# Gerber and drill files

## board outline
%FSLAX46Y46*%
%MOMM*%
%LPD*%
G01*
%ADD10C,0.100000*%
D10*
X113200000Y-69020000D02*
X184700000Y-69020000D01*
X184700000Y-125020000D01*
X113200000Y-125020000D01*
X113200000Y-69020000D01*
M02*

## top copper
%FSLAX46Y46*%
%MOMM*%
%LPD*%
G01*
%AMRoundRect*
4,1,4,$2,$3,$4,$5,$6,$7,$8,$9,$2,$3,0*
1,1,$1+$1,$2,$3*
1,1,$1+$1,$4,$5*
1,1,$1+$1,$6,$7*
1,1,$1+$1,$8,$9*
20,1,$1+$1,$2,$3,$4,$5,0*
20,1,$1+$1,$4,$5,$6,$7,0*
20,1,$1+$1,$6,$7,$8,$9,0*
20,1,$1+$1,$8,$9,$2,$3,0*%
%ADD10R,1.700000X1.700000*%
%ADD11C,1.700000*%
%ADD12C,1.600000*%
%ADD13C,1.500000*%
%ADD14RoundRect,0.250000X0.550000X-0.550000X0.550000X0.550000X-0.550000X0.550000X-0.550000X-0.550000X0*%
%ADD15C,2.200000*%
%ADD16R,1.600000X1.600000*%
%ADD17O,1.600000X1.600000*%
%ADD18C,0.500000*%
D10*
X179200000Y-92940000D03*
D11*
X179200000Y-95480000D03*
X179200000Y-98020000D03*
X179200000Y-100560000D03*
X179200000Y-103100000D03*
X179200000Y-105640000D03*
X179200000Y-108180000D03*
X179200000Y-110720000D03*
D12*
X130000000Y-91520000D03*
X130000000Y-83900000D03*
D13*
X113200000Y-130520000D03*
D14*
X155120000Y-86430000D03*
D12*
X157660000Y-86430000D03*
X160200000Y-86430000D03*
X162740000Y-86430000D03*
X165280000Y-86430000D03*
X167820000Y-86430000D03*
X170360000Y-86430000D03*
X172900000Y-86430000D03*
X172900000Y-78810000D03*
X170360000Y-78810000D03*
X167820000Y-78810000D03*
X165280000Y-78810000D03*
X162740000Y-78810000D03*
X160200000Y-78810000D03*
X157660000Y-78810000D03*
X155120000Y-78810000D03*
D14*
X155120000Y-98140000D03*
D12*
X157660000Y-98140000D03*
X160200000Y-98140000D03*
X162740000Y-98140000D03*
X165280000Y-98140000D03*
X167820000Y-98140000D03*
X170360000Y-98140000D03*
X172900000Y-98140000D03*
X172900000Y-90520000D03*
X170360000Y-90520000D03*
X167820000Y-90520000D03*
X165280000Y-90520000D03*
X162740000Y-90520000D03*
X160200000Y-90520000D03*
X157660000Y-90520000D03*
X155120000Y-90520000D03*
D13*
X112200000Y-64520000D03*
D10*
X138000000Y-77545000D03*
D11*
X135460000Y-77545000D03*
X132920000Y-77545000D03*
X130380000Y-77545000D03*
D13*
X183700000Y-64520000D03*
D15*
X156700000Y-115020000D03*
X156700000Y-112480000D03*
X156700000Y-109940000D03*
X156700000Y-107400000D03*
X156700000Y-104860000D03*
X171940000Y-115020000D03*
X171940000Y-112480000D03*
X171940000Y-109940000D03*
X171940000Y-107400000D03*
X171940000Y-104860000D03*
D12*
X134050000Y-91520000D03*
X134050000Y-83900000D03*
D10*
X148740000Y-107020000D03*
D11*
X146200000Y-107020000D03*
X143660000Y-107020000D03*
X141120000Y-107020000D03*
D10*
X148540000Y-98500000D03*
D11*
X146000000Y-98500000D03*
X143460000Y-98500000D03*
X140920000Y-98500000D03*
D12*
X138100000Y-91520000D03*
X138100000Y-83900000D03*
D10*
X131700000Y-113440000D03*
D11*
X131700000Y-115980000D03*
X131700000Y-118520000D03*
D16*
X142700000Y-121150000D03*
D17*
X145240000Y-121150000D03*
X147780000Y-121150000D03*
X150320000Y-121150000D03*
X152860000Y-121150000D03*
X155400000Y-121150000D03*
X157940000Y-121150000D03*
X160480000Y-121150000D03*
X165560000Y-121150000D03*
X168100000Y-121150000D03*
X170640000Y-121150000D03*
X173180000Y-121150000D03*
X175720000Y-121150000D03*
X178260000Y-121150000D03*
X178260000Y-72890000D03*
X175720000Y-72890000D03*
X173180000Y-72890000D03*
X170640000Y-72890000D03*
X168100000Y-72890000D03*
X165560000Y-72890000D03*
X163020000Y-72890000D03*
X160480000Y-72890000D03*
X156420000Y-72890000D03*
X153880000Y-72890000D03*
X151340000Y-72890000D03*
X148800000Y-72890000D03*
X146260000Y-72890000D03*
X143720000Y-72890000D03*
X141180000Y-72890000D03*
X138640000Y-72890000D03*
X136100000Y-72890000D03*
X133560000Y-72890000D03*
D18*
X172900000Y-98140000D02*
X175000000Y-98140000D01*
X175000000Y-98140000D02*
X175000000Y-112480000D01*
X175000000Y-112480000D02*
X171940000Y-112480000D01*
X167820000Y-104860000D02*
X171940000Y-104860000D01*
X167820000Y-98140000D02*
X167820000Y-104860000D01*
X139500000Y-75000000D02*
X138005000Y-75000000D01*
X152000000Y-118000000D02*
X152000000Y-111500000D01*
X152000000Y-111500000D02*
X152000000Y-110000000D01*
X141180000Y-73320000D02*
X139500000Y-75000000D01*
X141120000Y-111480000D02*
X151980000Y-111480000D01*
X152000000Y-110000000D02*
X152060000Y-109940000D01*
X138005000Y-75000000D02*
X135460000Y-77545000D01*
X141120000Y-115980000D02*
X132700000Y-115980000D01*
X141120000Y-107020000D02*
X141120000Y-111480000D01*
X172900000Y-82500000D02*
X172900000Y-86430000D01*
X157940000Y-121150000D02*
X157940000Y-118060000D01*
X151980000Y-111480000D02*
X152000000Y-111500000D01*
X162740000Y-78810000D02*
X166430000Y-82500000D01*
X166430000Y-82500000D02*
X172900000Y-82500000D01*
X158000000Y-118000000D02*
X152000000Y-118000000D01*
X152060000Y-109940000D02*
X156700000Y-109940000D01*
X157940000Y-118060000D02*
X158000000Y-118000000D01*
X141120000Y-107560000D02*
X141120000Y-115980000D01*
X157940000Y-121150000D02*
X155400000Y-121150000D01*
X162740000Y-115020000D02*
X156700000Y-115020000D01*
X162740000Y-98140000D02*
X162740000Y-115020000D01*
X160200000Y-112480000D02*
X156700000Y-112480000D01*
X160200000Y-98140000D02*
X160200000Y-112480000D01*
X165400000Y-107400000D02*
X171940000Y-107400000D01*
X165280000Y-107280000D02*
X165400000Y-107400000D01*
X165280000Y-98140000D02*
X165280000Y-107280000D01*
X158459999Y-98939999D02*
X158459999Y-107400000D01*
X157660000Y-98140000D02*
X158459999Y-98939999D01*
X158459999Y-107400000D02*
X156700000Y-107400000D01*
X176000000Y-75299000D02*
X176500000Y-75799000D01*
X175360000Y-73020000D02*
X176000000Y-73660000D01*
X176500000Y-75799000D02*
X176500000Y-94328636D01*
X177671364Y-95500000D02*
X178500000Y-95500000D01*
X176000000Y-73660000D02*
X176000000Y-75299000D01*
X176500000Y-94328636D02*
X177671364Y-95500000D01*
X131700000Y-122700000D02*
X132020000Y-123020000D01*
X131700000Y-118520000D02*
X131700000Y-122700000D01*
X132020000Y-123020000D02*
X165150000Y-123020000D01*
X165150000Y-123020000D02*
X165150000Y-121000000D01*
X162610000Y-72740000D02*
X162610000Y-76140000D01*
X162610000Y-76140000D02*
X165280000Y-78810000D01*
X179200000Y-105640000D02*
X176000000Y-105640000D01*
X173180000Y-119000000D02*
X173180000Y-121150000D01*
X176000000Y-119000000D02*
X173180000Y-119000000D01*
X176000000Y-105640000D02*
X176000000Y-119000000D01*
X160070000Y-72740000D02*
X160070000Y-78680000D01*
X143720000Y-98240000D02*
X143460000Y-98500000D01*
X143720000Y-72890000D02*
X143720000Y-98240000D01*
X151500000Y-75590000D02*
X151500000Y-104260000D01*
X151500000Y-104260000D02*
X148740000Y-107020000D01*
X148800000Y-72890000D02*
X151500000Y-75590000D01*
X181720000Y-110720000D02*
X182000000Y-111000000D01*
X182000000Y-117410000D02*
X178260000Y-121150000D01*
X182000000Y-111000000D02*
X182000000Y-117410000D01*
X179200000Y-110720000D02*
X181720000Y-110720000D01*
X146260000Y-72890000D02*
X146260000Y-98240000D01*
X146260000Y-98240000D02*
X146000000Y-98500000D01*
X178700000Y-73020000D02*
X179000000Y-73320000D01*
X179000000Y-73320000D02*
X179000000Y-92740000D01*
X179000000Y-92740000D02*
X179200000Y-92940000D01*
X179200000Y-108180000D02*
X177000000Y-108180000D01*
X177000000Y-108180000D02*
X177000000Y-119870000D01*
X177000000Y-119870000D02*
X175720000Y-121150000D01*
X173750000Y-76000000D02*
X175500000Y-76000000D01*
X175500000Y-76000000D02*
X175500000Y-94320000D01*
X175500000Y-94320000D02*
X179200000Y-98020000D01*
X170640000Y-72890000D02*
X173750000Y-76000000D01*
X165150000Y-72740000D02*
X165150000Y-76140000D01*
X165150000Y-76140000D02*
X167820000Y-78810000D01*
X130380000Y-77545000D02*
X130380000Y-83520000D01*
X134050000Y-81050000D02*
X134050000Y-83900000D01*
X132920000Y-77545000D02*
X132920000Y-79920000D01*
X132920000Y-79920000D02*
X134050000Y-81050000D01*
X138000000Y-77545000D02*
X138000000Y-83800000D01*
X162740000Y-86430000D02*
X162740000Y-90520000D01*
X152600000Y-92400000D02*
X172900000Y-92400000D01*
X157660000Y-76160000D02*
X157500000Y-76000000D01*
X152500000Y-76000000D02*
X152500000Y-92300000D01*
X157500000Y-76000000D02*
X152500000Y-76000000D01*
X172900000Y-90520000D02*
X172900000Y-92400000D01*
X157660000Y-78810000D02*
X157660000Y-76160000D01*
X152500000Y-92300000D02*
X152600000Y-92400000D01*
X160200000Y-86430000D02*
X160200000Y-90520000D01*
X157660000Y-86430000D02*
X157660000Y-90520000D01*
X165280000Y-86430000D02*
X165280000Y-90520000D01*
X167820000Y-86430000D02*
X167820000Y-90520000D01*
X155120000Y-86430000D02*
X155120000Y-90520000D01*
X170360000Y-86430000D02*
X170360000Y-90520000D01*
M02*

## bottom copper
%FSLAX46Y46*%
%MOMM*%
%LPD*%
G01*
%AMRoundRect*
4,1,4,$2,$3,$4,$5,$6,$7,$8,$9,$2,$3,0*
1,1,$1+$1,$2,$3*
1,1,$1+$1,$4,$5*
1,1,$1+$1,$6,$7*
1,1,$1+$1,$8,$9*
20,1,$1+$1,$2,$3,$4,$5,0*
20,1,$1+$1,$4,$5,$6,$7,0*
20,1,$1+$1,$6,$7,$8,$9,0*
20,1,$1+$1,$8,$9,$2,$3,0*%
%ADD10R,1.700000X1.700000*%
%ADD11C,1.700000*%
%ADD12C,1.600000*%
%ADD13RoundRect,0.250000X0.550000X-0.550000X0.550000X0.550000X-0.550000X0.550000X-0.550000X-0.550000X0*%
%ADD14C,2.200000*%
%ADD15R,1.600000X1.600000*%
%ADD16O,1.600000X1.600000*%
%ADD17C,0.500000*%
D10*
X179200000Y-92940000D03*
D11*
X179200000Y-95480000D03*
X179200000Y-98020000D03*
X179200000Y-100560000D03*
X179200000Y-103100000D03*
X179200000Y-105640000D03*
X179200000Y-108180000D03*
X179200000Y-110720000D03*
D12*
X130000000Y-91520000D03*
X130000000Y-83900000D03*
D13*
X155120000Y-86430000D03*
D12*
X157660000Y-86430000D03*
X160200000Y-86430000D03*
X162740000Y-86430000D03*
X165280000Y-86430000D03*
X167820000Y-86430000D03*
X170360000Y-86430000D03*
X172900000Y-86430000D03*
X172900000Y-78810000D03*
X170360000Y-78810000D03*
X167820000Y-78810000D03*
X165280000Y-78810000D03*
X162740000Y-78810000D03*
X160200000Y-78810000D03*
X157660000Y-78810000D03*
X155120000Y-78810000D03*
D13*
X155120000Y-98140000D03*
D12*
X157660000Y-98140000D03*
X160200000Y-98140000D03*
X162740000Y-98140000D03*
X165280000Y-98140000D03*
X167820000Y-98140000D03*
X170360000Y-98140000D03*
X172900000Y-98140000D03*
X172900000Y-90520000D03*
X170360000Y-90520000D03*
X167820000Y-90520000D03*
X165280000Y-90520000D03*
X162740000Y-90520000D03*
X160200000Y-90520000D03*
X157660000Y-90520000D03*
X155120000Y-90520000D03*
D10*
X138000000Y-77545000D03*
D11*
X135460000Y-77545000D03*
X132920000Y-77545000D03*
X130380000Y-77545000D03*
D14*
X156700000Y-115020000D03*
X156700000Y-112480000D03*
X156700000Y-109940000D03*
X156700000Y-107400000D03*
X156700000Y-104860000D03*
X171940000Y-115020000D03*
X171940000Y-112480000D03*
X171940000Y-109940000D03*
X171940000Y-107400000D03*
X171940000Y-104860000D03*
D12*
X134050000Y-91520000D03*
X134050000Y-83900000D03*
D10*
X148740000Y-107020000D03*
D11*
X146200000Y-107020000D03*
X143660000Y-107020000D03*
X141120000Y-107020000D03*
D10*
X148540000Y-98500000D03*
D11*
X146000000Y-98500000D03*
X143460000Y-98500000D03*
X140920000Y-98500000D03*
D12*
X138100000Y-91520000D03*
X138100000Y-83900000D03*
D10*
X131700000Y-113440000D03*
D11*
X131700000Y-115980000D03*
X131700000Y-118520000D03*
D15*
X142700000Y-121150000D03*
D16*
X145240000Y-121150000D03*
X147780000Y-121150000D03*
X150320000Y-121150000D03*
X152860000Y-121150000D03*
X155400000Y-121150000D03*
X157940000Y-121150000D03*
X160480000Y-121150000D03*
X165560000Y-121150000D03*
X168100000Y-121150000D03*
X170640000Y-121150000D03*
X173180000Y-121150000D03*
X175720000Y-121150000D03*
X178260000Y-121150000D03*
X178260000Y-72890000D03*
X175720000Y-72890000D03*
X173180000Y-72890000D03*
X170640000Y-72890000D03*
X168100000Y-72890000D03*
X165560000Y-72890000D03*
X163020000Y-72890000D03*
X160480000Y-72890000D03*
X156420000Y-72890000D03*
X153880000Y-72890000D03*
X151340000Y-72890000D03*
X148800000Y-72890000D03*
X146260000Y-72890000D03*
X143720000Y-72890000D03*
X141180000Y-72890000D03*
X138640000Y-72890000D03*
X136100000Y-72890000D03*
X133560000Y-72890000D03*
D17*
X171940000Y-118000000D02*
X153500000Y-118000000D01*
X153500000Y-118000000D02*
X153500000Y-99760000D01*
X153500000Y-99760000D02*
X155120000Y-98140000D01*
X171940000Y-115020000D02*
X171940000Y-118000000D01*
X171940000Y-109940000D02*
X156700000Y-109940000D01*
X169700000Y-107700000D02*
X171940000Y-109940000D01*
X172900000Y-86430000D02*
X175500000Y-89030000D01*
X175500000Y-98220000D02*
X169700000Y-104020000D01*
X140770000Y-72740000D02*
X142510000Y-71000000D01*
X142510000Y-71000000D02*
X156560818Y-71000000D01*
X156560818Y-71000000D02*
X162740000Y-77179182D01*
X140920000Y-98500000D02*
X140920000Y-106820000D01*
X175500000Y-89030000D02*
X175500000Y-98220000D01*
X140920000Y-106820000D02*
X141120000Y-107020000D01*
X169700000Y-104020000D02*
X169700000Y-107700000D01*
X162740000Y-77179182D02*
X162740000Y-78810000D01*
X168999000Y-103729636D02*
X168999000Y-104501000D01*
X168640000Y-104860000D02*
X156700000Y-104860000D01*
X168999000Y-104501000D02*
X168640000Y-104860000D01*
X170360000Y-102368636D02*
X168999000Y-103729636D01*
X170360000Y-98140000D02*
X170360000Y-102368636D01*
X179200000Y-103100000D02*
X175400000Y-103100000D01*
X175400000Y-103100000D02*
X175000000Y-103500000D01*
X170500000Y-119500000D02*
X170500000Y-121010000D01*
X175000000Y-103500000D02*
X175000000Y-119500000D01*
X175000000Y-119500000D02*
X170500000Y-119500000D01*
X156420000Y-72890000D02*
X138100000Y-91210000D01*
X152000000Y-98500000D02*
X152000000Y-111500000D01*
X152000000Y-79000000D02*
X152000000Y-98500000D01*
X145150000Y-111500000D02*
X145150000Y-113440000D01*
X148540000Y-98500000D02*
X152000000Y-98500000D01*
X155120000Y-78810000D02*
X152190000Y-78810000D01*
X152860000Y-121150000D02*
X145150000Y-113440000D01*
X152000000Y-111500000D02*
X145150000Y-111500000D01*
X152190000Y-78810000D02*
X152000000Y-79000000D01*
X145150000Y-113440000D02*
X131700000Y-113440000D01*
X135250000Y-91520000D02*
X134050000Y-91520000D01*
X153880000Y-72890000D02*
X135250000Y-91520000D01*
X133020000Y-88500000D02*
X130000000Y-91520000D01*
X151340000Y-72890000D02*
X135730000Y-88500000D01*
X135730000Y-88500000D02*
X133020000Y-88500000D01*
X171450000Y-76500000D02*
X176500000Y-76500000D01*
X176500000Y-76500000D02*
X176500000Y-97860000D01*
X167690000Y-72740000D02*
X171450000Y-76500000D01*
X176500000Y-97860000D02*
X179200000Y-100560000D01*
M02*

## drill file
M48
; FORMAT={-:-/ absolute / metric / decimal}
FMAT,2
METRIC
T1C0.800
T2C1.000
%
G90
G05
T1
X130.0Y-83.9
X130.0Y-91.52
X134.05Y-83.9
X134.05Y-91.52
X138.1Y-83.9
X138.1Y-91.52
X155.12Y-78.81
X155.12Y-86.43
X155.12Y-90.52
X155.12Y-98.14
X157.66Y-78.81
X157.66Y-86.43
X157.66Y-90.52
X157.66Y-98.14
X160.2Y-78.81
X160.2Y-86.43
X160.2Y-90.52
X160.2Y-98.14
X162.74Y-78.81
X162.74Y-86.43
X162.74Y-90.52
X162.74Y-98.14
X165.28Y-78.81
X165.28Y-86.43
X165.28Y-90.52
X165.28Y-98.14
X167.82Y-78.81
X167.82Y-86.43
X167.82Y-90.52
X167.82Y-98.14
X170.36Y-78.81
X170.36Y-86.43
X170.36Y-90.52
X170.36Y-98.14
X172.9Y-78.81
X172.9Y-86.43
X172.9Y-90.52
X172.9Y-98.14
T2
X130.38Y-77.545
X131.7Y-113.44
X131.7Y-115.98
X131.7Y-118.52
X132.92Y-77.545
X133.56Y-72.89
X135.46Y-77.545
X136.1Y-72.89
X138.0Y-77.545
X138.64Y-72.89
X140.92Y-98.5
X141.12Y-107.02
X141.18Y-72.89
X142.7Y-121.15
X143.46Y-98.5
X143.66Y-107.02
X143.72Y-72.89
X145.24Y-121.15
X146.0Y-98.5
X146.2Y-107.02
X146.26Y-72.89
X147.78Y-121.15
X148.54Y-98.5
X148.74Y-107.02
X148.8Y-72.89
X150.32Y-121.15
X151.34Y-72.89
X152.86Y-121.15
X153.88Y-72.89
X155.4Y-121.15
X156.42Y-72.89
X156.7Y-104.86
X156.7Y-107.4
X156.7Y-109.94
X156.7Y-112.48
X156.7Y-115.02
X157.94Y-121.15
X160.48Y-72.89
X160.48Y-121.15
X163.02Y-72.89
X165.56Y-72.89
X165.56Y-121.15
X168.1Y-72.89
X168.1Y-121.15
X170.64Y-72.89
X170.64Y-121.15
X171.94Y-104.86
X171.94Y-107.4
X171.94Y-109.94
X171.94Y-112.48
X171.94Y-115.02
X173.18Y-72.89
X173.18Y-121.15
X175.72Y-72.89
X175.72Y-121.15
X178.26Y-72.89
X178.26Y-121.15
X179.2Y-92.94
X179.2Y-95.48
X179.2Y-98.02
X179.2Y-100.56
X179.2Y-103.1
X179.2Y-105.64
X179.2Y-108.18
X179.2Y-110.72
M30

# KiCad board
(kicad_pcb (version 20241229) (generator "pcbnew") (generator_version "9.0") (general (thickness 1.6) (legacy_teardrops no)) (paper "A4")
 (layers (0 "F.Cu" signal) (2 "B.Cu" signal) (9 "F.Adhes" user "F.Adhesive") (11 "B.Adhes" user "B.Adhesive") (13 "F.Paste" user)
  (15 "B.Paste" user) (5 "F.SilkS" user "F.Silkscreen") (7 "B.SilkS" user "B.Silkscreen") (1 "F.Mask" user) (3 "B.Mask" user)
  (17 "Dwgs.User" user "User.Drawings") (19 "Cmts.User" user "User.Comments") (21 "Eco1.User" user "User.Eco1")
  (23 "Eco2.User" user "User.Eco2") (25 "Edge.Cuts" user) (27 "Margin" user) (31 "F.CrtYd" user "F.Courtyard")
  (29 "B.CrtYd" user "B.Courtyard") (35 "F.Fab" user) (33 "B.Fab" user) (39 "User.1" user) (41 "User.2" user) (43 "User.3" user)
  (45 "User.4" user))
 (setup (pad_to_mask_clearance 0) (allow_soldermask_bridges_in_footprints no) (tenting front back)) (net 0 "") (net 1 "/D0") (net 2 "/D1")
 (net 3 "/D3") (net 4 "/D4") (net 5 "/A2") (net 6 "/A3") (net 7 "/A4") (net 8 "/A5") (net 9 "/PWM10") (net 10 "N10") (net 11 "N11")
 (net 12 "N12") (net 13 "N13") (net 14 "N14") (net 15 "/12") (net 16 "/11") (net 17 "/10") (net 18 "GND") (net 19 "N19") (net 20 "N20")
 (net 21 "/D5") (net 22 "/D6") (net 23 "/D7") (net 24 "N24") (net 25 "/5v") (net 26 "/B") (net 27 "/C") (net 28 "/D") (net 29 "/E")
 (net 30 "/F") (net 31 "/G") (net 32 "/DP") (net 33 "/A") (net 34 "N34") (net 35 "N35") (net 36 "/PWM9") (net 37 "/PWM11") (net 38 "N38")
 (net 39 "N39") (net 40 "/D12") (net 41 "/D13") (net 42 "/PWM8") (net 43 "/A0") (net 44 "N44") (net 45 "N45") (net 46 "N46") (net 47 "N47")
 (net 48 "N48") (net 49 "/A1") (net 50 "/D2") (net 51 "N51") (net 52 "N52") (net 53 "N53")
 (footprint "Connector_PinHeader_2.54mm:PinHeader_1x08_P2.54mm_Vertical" (layer "F.Cu") (at 179.2 92.94)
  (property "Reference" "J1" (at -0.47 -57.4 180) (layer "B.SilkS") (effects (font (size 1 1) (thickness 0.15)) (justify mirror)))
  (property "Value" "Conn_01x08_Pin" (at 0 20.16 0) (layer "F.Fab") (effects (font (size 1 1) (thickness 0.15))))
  (pad "1" thru_hole rect (at 0 0) (size 1.7 1.7) (drill 1) (layers "*.Cu" "*.Mask") (remove_unused_layers no) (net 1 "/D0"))
  (pad "2" thru_hole circle (at 0 2.54) (size 1.7 1.7) (drill 1) (layers "*.Cu" "*.Mask") (remove_unused_layers no) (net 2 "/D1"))
  (pad "3" thru_hole circle (at 0 5.08) (size 1.7 1.7) (drill 1) (layers "*.Cu" "*.Mask") (remove_unused_layers no) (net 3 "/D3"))
  (pad "4" thru_hole circle (at 0 7.62) (size 1.7 1.7) (drill 1) (layers "*.Cu" "*.Mask") (remove_unused_layers no) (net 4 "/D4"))
  (pad "5" thru_hole circle (at 0 10.16) (size 1.7 1.7) (drill 1) (layers "*.Cu" "*.Mask") (remove_unused_layers no) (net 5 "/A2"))
  (pad "6" thru_hole circle (at 0 12.7) (size 1.7 1.7) (drill 1) (layers "*.Cu" "*.Mask") (remove_unused_layers no) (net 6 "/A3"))
  (pad "7" thru_hole circle (at 0 15.24) (size 1.7 1.7) (drill 1) (layers "*.Cu" "*.Mask") (remove_unused_layers no) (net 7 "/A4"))
  (pad "8" thru_hole circle (at 0 17.78) (size 1.7 1.7) (drill 1) (layers "*.Cu" "*.Mask") (remove_unused_layers no) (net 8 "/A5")))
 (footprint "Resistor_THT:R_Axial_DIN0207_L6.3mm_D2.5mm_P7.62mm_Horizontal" (layer "F.Cu") (at 130 91.52 90)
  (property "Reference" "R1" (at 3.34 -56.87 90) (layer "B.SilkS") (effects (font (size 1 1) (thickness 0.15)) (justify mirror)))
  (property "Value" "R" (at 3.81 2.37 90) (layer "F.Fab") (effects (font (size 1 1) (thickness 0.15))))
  (pad "1" thru_hole circle (at 0 0 90) (size 1.6 1.6) (drill 0.8) (layers "*.Cu" "*.Mask") (remove_unused_layers no) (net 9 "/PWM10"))
  (pad "2" thru_hole circle (at 7.62 0 90) (size 1.6 1.6) (drill 0.8) (layers "*.Cu" "*.Mask") (remove_unused_layers no) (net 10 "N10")))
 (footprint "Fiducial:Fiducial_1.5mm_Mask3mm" (layer "F.Cu") (at 113.2 130.52)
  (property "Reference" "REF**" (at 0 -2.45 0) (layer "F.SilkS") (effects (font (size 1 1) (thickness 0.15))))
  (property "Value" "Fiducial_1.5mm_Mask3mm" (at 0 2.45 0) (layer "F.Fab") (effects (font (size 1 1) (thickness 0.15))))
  (pad "" smd circle (at 0 0) (size 1.5 1.5) (layers "F.Cu" "F.Mask") (solder_mask_margin 0.75)))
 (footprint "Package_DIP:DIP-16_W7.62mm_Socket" (layer "F.Cu") (at 155.12 86.43 90)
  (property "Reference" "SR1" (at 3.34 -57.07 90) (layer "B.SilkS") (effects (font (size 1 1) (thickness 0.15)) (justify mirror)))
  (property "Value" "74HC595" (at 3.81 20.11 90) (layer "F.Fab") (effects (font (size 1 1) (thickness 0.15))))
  (pad "1" thru_hole roundrect (at 0 0 90) (size 1.6 1.6) (drill 0.8) (layers "*.Cu" "*.Mask") (remove_unused_layers no)
   (roundrect_rratio 0.15625) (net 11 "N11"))
  (pad "2" thru_hole circle (at 0 2.54 90) (size 1.6 1.6) (drill 0.8) (layers "*.Cu" "*.Mask") (remove_unused_layers no) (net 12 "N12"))
  (pad "3" thru_hole circle (at 0 5.08 90) (size 1.6 1.6) (drill 0.8) (layers "*.Cu" "*.Mask") (remove_unused_layers no) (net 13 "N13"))
  (pad "4" thru_hole circle (at 0 7.62 90) (size 1.6 1.6) (drill 0.8) (layers "*.Cu" "*.Mask") (remove_unused_layers no) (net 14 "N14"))
  (pad "5" thru_hole circle (at 0 10.16 90) (size 1.6 1.6) (drill 0.8) (layers "*.Cu" "*.Mask") (remove_unused_layers no) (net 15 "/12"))
  (pad "6" thru_hole circle (at 0 12.7 90) (size 1.6 1.6) (drill 0.8) (layers "*.Cu" "*.Mask") (remove_unused_layers no) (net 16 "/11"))
  (pad "7" thru_hole circle (at 0 15.24 90) (size 1.6 1.6) (drill 0.8) (layers "*.Cu" "*.Mask") (remove_unused_layers no) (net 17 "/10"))
  (pad "8" thru_hole circle (at 0 17.78 90) (size 1.6 1.6) (drill 0.8) (layers "*.Cu" "*.Mask") (remove_unused_layers no) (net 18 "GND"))
  (pad "9" thru_hole circle (at 7.62 17.78 90) (size 1.6 1.6) (drill 0.8) (layers "*.Cu" "*.Mask") (remove_unused_layers no) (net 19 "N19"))
  (pad "10" thru_hole circle (at 7.62 15.24 90) (size 1.6 1.6) (drill 0.8) (layers "*.Cu" "*.Mask") (remove_unused_layers no) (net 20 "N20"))
  (pad "11" thru_hole circle (at 7.62 12.7 90) (size 1.6 1.6) (drill 0.8) (layers "*.Cu" "*.Mask") (remove_unused_layers no) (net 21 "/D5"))
  (pad "12" thru_hole circle (at 7.62 10.16 90) (size 1.6 1.6) (drill 0.8) (layers "*.Cu" "*.Mask") (remove_unused_layers no) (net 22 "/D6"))
  (pad "13" thru_hole circle (at 7.62 7.62 90) (size 1.6 1.6) (drill 0.8) (layers "*.Cu" "*.Mask") (remove_unused_layers no) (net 18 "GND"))
  (pad "14" thru_hole circle (at 7.62 5.08 90) (size 1.6 1.6) (drill 0.8) (layers "*.Cu" "*.Mask") (remove_unused_layers no) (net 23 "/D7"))
  (pad "15" thru_hole circle (at 7.62 2.54 90) (size 1.6 1.6) (drill 0.8) (layers "*.Cu" "*.Mask") (remove_unused_layers no) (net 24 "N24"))
  (pad "16" thru_hole circle (at 7.62 0 90) (size 1.6 1.6) (drill 0.8) (layers "*.Cu" "*.Mask") (remove_unused_layers no) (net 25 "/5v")))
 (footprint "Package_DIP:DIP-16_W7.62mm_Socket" (layer "F.Cu") (at 155.12 98.14 90)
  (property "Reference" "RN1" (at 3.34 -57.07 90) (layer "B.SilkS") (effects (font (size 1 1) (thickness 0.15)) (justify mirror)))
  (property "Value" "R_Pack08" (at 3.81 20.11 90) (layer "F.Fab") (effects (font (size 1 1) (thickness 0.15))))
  (pad "1" thru_hole roundrect (at 0 0 90) (size 1.6 1.6) (drill 0.8) (layers "*.Cu" "*.Mask") (remove_unused_layers no)
   (roundrect_rratio 0.15625) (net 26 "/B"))
  (pad "2" thru_hole circle (at 0 2.54 90) (size 1.6 1.6) (drill 0.8) (layers "*.Cu" "*.Mask") (remove_unused_layers no) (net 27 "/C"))
  (pad "3" thru_hole circle (at 0 5.08 90) (size 1.6 1.6) (drill 0.8) (layers "*.Cu" "*.Mask") (remove_unused_layers no) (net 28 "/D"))
  (pad "4" thru_hole circle (at 0 7.62 90) (size 1.6 1.6) (drill 0.8) (layers "*.Cu" "*.Mask") (remove_unused_layers no) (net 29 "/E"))
  (pad "5" thru_hole circle (at 0 10.16 90) (size 1.6 1.6) (drill 0.8) (layers "*.Cu" "*.Mask") (remove_unused_layers no) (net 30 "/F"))
  (pad "6" thru_hole circle (at 0 12.7 90) (size 1.6 1.6) (drill 0.8) (layers "*.Cu" "*.Mask") (remove_unused_layers no) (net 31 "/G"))
  (pad "7" thru_hole circle (at 0 15.24 90) (size 1.6 1.6) (drill 0.8) (layers "*.Cu" "*.Mask") (remove_unused_layers no) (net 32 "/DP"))
  (pad "8" thru_hole circle (at 0 17.78 90) (size 1.6 1.6) (drill 0.8) (layers "*.Cu" "*.Mask") (remove_unused_layers no) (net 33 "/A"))
  (pad "9" thru_hole circle (at 7.62 17.78 90) (size 1.6 1.6) (drill 0.8) (layers "*.Cu" "*.Mask") (remove_unused_layers no) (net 24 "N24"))
  (pad "10" thru_hole circle (at 7.62 15.24 90) (size 1.6 1.6) (drill 0.8) (layers "*.Cu" "*.Mask") (remove_unused_layers no) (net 17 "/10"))
  (pad "11" thru_hole circle (at 7.62 12.7 90) (size 1.6 1.6) (drill 0.8) (layers "*.Cu" "*.Mask") (remove_unused_layers no) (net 16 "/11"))
  (pad "12" thru_hole circle (at 7.62 10.16 90) (size 1.6 1.6) (drill 0.8) (layers "*.Cu" "*.Mask") (remove_unused_layers no) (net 15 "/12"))
  (pad "13" thru_hole circle (at 7.62 7.62 90) (size 1.6 1.6) (drill 0.8) (layers "*.Cu" "*.Mask") (remove_unused_layers no) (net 14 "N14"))
  (pad "14" thru_hole circle (at 7.62 5.08 90) (size 1.6 1.6) (drill 0.8) (layers "*.Cu" "*.Mask") (remove_unused_layers no) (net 13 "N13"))
  (pad "15" thru_hole circle (at 7.62 2.54 90) (size 1.6 1.6) (drill 0.8) (layers "*.Cu" "*.Mask") (remove_unused_layers no) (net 12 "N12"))
  (pad "16" thru_hole circle (at 7.62 0 90) (size 1.6 1.6) (drill 0.8) (layers "*.Cu" "*.Mask") (remove_unused_layers no) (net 11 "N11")))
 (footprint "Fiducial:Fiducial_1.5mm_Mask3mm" (layer "F.Cu") (at 112.2 64.52)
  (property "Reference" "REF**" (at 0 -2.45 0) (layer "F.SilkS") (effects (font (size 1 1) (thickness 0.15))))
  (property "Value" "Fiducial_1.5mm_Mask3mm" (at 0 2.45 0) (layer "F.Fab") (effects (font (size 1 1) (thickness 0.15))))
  (pad "" smd circle (at 0 0) (size 1.5 1.5) (layers "F.Cu" "F.Mask") (solder_mask_margin 0.75)))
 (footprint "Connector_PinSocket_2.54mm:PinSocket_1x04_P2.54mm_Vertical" (layer "F.Cu") (at 138 77.545 -90)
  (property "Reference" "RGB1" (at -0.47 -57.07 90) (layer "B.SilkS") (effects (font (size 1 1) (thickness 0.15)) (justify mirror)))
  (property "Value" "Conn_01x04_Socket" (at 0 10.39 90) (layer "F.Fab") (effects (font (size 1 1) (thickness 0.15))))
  (pad "1" thru_hole rect (at 0 0 270) (size 1.7 1.7) (drill 1) (layers "*.Cu" "*.Mask") (remove_unused_layers no) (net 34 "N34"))
  (pad "2" thru_hole circle (at 0 2.54 270) (size 1.7 1.7) (drill 1) (layers "*.Cu" "*.Mask") (remove_unused_layers no) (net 18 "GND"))
  (pad "3" thru_hole circle (at 0 5.08 270) (size 1.7 1.7) (drill 1) (layers "*.Cu" "*.Mask") (remove_unused_layers no) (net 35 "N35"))
  (pad "4" thru_hole circle (at 0 7.62 270) (size 1.7 1.7) (drill 1) (layers "*.Cu" "*.Mask") (remove_unused_layers no) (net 10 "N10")))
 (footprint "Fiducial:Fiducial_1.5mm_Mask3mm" (layer "F.Cu") (at 183.7 64.52)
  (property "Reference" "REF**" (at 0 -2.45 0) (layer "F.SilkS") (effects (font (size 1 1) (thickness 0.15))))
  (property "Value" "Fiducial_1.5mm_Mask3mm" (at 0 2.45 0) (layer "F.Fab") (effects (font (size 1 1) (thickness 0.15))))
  (pad "" smd circle (at 0 0) (size 1.5 1.5) (layers "F.Cu" "F.Mask") (solder_mask_margin 0.75)))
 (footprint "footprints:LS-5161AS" (layer "F.Cu") (at 156.7 115.02 90)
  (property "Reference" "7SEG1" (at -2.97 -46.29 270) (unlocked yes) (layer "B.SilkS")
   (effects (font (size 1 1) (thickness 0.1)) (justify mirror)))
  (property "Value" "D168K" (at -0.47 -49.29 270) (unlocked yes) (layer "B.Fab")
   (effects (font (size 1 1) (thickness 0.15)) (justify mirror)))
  (pad "1" thru_hole circle (at 0 0 90) (size 2.2 2.2) (drill 1) (layers "*.Cu" "*.Mask") (remove_unused_layers no) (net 29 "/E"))
  (pad "2" thru_hole circle (at 2.54 0 90) (size 2.2 2.2) (drill 1) (layers "*.Cu" "*.Mask") (remove_unused_layers no) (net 28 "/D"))
  (pad "3" thru_hole circle (at 5.08 0 90) (size 2.2 2.2) (drill 1) (layers "*.Cu" "*.Mask") (remove_unused_layers no) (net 18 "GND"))
  (pad "4" thru_hole circle (at 7.62 0 90) (size 2.2 2.2) (drill 1) (layers "*.Cu" "*.Mask") (remove_unused_layers no) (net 27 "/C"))
  (pad "5" thru_hole circle (at 10.16 0 90) (size 2.2 2.2) (drill 1) (layers "*.Cu" "*.Mask") (remove_unused_layers no) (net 32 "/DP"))
  (pad "6" thru_hole circle (at 0 15.24 90) (size 2.2 2.2) (drill 1) (layers "*.Cu" "*.Mask") (remove_unused_layers no) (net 26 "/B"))
  (pad "7" thru_hole circle (at 2.54 15.24 90) (size 2.2 2.2) (drill 1) (layers "*.Cu" "*.Mask") (remove_unused_layers no) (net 33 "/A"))
  (pad "8" thru_hole circle (at 5.08 15.24 90) (size 2.2 2.2) (drill 1) (layers "*.Cu" "*.Mask") (remove_unused_layers no) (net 18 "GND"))
  (pad "9" thru_hole circle (at 7.62 15.24 90) (size 2.2 2.2) (drill 1) (layers "*.Cu" "*.Mask") (remove_unused_layers no) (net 30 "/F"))
  (pad "10" thru_hole circle (at 10.16 15.24 90) (size 2.2 2.2) (drill 1) (layers "*.Cu" "*.Mask") (remove_unused_layers no) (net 31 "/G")))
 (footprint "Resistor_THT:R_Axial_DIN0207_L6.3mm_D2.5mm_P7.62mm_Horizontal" (layer "F.Cu") (at 134.05 91.52 90)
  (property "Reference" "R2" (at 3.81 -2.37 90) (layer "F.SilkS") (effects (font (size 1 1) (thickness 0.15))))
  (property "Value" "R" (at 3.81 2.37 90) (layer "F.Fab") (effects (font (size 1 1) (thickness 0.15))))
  (pad "1" thru_hole circle (at 0 0 90) (size 1.6 1.6) (drill 0.8) (layers "*.Cu" "*.Mask") (remove_unused_layers no) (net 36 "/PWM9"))
  (pad "2" thru_hole circle (at 7.62 0 90) (size 1.6 1.6) (drill 0.8) (layers "*.Cu" "*.Mask") (remove_unused_layers no) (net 35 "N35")))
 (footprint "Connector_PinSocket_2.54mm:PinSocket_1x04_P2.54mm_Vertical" (layer "F.Cu") (at 148.74 107.02 -90)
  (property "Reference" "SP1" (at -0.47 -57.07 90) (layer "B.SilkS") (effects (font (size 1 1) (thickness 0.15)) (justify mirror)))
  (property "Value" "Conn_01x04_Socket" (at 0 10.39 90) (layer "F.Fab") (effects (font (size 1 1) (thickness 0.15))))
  (pad "1" thru_hole rect (at 0 0 270) (size 1.7 1.7) (drill 1) (layers "*.Cu" "*.Mask") (remove_unused_layers no) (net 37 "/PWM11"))
  (pad "2" thru_hole circle (at 0 2.54 270) (size 1.7 1.7) (drill 1) (layers "*.Cu" "*.Mask") (remove_unused_layers no) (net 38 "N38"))
  (pad "3" thru_hole circle (at 0 5.08 270) (size 1.7 1.7) (drill 1) (layers "*.Cu" "*.Mask") (remove_unused_layers no) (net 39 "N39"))
  (pad "4" thru_hole circle (at 0 7.62 270) (size 1.7 1.7) (drill 1) (layers "*.Cu" "*.Mask") (remove_unused_layers no) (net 18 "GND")))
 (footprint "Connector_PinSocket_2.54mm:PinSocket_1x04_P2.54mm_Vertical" (layer "F.Cu") (at 148.54 98.5 -90)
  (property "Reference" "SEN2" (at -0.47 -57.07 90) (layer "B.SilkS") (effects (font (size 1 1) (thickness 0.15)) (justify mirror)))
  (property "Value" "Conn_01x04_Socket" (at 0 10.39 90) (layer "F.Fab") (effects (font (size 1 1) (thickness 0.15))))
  (pad "1" thru_hole rect (at 0 0 270) (size 1.7 1.7) (drill 1) (layers "*.Cu" "*.Mask") (remove_unused_layers no) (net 25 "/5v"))
  (pad "2" thru_hole circle (at 0 2.54 270) (size 1.7 1.7) (drill 1) (layers "*.Cu" "*.Mask") (remove_unused_layers no) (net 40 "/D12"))
  (pad "3" thru_hole circle (at 0 5.08 270) (size 1.7 1.7) (drill 1) (layers "*.Cu" "*.Mask") (remove_unused_layers no) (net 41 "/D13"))
  (pad "4" thru_hole circle (at 0 7.62 270) (size 1.7 1.7) (drill 1) (layers "*.Cu" "*.Mask") (remove_unused_layers no) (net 18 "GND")))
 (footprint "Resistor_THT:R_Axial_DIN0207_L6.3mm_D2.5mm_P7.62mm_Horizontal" (layer "F.Cu") (at 138.1 91.52 90)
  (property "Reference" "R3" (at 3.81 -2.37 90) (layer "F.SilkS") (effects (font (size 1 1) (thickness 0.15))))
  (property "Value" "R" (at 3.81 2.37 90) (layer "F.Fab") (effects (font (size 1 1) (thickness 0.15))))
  (pad "1" thru_hole circle (at 0 0 90) (size 1.6 1.6) (drill 0.8) (layers "*.Cu" "*.Mask") (remove_unused_layers no) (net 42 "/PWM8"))
  (pad "2" thru_hole circle (at 7.62 0 90) (size 1.6 1.6) (drill 0.8) (layers "*.Cu" "*.Mask") (remove_unused_layers no) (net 34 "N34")))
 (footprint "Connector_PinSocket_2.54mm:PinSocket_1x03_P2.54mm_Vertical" (layer "F.Cu") (at 131.7 113.44)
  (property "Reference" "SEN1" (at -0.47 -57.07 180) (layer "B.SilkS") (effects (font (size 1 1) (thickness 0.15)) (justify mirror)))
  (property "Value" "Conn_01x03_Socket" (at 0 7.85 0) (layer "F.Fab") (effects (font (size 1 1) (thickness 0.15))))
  (pad "1" thru_hole rect (at 0 0) (size 1.7 1.7) (drill 1) (layers "*.Cu" "*.Mask") (remove_unused_layers no) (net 25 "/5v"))
  (pad "2" thru_hole circle (at 0 2.54) (size 1.7 1.7) (drill 1) (layers "*.Cu" "*.Mask") (remove_unused_layers no) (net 18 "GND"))
  (pad "3" thru_hole circle (at 0 5.08) (size 1.7 1.7) (drill 1) (layers "*.Cu" "*.Mask") (remove_unused_layers no) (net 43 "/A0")))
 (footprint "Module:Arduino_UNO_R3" (layer "B.Cu") (at 142.7 121.15)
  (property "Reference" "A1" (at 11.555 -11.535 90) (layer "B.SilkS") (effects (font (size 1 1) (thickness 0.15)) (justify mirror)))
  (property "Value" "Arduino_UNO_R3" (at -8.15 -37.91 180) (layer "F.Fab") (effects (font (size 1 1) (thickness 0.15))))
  (pad "1" thru_hole rect (at 0 0 270) (size 1.6 1.6) (drill 1) (layers "*.Cu" "*.Mask") (remove_unused_layers no) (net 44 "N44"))
  (pad "2" thru_hole oval (at 2.54 0 270) (size 1.6 1.6) (drill 1) (layers "*.Cu" "*.Mask") (remove_unused_layers no) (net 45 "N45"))
  (pad "3" thru_hole oval (at 5.08 0 270) (size 1.6 1.6) (drill 1) (layers "*.Cu" "*.Mask") (remove_unused_layers no) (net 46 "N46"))
  (pad "4" thru_hole oval (at 7.62 0 270) (size 1.6 1.6) (drill 1) (layers "*.Cu" "*.Mask") (remove_unused_layers no) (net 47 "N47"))
  (pad "5" thru_hole oval (at 10.16 0 270) (size 1.6 1.6) (drill 1) (layers "*.Cu" "*.Mask") (remove_unused_layers no) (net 25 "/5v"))
  (pad "6" thru_hole oval (at 12.7 0 270) (size 1.6 1.6) (drill 1) (layers "*.Cu" "*.Mask") (remove_unused_layers no) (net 18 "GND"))
  (pad "7" thru_hole oval (at 15.24 0 270) (size 1.6 1.6) (drill 1) (layers "*.Cu" "*.Mask") (remove_unused_layers no) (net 18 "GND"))
  (pad "8" thru_hole oval (at 17.78 0 270) (size 1.6 1.6) (drill 1) (layers "*.Cu" "*.Mask") (remove_unused_layers no) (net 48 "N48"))
  (pad "9" thru_hole oval (at 22.86 0 270) (size 1.6 1.6) (drill 1) (layers "*.Cu" "*.Mask") (remove_unused_layers no) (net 43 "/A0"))
  (pad "10" thru_hole oval (at 25.4 0 270) (size 1.6 1.6) (drill 1) (layers "*.Cu" "*.Mask") (remove_unused_layers no) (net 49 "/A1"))
  (pad "11" thru_hole oval (at 27.94 0 270) (size 1.6 1.6) (drill 1) (layers "*.Cu" "*.Mask") (remove_unused_layers no) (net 5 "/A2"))
  (pad "12" thru_hole oval (at 30.48 0 270) (size 1.6 1.6) (drill 1) (layers "*.Cu" "*.Mask") (remove_unused_layers no) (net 6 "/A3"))
  (pad "13" thru_hole oval (at 33.02 0 270) (size 1.6 1.6) (drill 1) (layers "*.Cu" "*.Mask") (remove_unused_layers no) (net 7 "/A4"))
  (pad "14" thru_hole oval (at 35.56 0 270) (size 1.6 1.6) (drill 1) (layers "*.Cu" "*.Mask") (remove_unused_layers no) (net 8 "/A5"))
  (pad "15" thru_hole oval (at 35.56 -48.26 270) (size 1.6 1.6) (drill 1) (layers "*.Cu" "*.Mask") (remove_unused_layers no) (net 1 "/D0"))
  (pad "16" thru_hole oval (at 33.02 -48.26 270) (size 1.6 1.6) (drill 1) (layers "*.Cu" "*.Mask") (remove_unused_layers no) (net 2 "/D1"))
  (pad "17" thru_hole oval (at 30.48 -48.26 270) (size 1.6 1.6) (drill 1) (layers "*.Cu" "*.Mask") (remove_unused_layers no) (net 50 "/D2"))
  (pad "18" thru_hole oval (at 27.94 -48.26 270) (size 1.6 1.6) (drill 1) (layers "*.Cu" "*.Mask") (remove_unused_layers no) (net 3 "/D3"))
  (pad "19" thru_hole oval (at 25.4 -48.26 270) (size 1.6 1.6) (drill 1) (layers "*.Cu" "*.Mask") (remove_unused_layers no) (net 4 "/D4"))
  (pad "20" thru_hole oval (at 22.86 -48.26 270) (size 1.6 1.6) (drill 1) (layers "*.Cu" "*.Mask") (remove_unused_layers no) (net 21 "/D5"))
  (pad "21" thru_hole oval (at 20.32 -48.26 270) (size 1.6 1.6) (drill 1) (layers "*.Cu" "*.Mask") (remove_unused_layers no) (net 22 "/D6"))
  (pad "22" thru_hole oval (at 17.78 -48.26 270) (size 1.6 1.6) (drill 1) (layers "*.Cu" "*.Mask") (remove_unused_layers no) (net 23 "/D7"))
  (pad "23" thru_hole oval (at 13.72 -48.26 270) (size 1.6 1.6) (drill 1) (layers "*.Cu" "*.Mask") (remove_unused_layers no)
   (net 42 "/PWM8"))
  (pad "24" thru_hole oval (at 11.18 -48.26 270) (size 1.6 1.6) (drill 1) (layers "*.Cu" "*.Mask") (remove_unused_layers no)
   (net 36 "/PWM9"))
  (pad "25" thru_hole oval (at 8.64 -48.26 270) (size 1.6 1.6) (drill 1) (layers "*.Cu" "*.Mask") (remove_unused_layers no) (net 9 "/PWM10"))
  (pad "26" thru_hole oval (at 6.1 -48.26 270) (size 1.6 1.6) (drill 1) (layers "*.Cu" "*.Mask") (remove_unused_layers no) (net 37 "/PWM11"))
  (pad "27" thru_hole oval (at 3.56 -48.26 270) (size 1.6 1.6) (drill 1) (layers "*.Cu" "*.Mask") (remove_unused_layers no) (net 40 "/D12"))
  (pad "28" thru_hole oval (at 1.02 -48.26 270) (size 1.6 1.6) (drill 1) (layers "*.Cu" "*.Mask") (remove_unused_layers no) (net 41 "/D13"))
  (pad "29" thru_hole oval (at -1.52 -48.26 270) (size 1.6 1.6) (drill 1) (layers "*.Cu" "*.Mask") (remove_unused_layers no) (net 18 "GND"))
  (pad "30" thru_hole oval (at -4.06 -48.26 270) (size 1.6 1.6) (drill 1) (layers "*.Cu" "*.Mask") (remove_unused_layers no) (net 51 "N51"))
  (pad "31" thru_hole oval (at -6.6 -48.26 270) (size 1.6 1.6) (drill 1) (layers "*.Cu" "*.Mask") (remove_unused_layers no) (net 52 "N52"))
  (pad "32" thru_hole oval (at -9.14 -48.26 270) (size 1.6 1.6) (drill 1) (layers "*.Cu" "*.Mask") (remove_unused_layers no) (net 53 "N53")))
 (gr_rect (start 113.2 69.02) (end 184.7 125.02) (stroke (width 0.1) (type default)) (fill no) (layer "Edge.Cuts"))
 (segment (start 171.94 118) (end 153.5 118) (width 0.5) (layer "B.Cu") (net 26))
 (segment (start 153.5 118) (end 153.5 99.76) (width 0.5) (layer "B.Cu") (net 26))
 (segment (start 153.5 99.76) (end 155.12 98.14) (width 0.5) (layer "B.Cu") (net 26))
 (segment (start 171.94 115.02) (end 171.94 118) (width 0.5) (layer "B.Cu") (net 26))
 (segment (start 172.9 98.14) (end 175 98.14) (width 0.5) (layer "F.Cu") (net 33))
 (segment (start 175 98.14) (end 175 112.48) (width 0.5) (layer "F.Cu") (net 33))
 (segment (start 175 112.48) (end 171.94 112.48) (width 0.5) (layer "F.Cu") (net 33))
 (segment (start 167.82 104.86) (end 171.94 104.86) (width 0.5) (layer "F.Cu") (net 31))
 (segment (start 167.82 98.14) (end 167.82 104.86) (width 0.5) (layer "F.Cu") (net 31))
 (segment (start 139.5 75) (end 138.005 75) (width 0.5) (layer "F.Cu") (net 18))
 (segment (start 152 118) (end 152 111.5) (width 0.5) (layer "F.Cu") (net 18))
 (segment (start 152 111.5) (end 152 110) (width 0.5) (layer "F.Cu") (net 18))
 (segment (start 141.18 73.32) (end 139.5 75) (width 0.5) (layer "F.Cu") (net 18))
 (segment (start 141.12 111.48) (end 151.98 111.48) (width 0.5) (layer "F.Cu") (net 18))
 (segment (start 152 110) (end 152.06 109.94) (width 0.5) (layer "F.Cu") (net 18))
 (segment (start 138.005 75) (end 135.46 77.545) (width 0.5) (layer "F.Cu") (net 18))
 (segment (start 141.12 115.98) (end 132.7 115.98) (width 0.5) (layer "F.Cu") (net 18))
 (segment (start 141.12 107.02) (end 141.12 111.48) (width 0.5) (layer "F.Cu") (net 18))
 (segment (start 172.9 82.5) (end 172.9 86.43) (width 0.5) (layer "F.Cu") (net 18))
 (segment (start 157.94 121.15) (end 157.94 118.06) (width 0.5) (layer "F.Cu") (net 18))
 (segment (start 151.98 111.48) (end 152 111.5) (width 0.5) (layer "F.Cu") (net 18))
 (segment (start 162.74 78.81) (end 166.43 82.5) (width 0.5) (layer "F.Cu") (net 18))
 (segment (start 166.43 82.5) (end 172.9 82.5) (width 0.5) (layer "F.Cu") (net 18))
 (segment (start 158 118) (end 152 118) (width 0.5) (layer "F.Cu") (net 18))
 (segment (start 152.06 109.94) (end 156.7 109.94) (width 0.5) (layer "F.Cu") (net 18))
 (segment (start 157.94 118.06) (end 158 118) (width 0.5) (layer "F.Cu") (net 18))
 (segment (start 141.12 107.56) (end 141.12 115.98) (width 0.5) (layer "F.Cu") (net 18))
 (segment (start 157.94 121.15) (end 155.4 121.15) (width 0.5) (layer "F.Cu") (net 18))
 (segment (start 171.94 109.94) (end 156.7 109.94) (width 0.5) (layer "B.Cu") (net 18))
 (segment (start 169.7 107.7) (end 171.94 109.94) (width 0.5) (layer "B.Cu") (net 18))
 (segment (start 172.9 86.43) (end 175.5 89.03) (width 0.5) (layer "B.Cu") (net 18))
 (segment (start 175.5 98.22) (end 169.7 104.02) (width 0.5) (layer "B.Cu") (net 18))
 (segment (start 140.77 72.74) (end 142.51 71) (width 0.5) (layer "B.Cu") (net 18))
 (segment (start 142.51 71) (end 156.560818 71) (width 0.5) (layer "B.Cu") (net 18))
 (segment (start 156.560818 71) (end 162.74 77.179182) (width 0.5) (layer "B.Cu") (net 18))
 (segment (start 140.92 98.5) (end 140.92 106.82) (width 0.5) (layer "B.Cu") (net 18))
 (segment (start 175.5 89.03) (end 175.5 98.22) (width 0.5) (layer "B.Cu") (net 18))
 (segment (start 140.92 106.82) (end 141.12 107.02) (width 0.5) (layer "B.Cu") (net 18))
 (segment (start 169.7 104.02) (end 169.7 107.7) (width 0.5) (layer "B.Cu") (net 18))
 (segment (start 162.74 77.179182) (end 162.74 78.81) (width 0.5) (layer "B.Cu") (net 18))
 (segment (start 162.74 115.02) (end 156.7 115.02) (width 0.5) (layer "F.Cu") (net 29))
 (segment (start 162.74 98.14) (end 162.74 115.02) (width 0.5) (layer "F.Cu") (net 29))
 (segment (start 160.2 112.48) (end 156.7 112.48) (width 0.5) (layer "F.Cu") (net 28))
 (segment (start 160.2 98.14) (end 160.2 112.48) (width 0.5) (layer "F.Cu") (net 28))
 (segment (start 165.4 107.4) (end 171.94 107.4) (width 0.5) (layer "F.Cu") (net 30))
 (segment (start 165.28 107.28) (end 165.4 107.4) (width 0.5) (layer "F.Cu") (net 30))
 (segment (start 165.28 98.14) (end 165.28 107.28) (width 0.5) (layer "F.Cu") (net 30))
 (segment (start 168.999 103.729636) (end 168.999 104.501) (width 0.5) (layer "B.Cu") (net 32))
 (segment (start 168.64 104.86) (end 156.7 104.86) (width 0.5) (layer "B.Cu") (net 32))
 (segment (start 168.999 104.501) (end 168.64 104.86) (width 0.5) (layer "B.Cu") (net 32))
 (segment (start 170.36 102.368636) (end 168.999 103.729636) (width 0.5) (layer "B.Cu") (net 32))
 (segment (start 170.36 98.14) (end 170.36 102.368636) (width 0.5) (layer "B.Cu") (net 32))
 (segment (start 158.459999 98.939999) (end 158.459999 107.4) (width 0.5) (layer "F.Cu") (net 27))
 (segment (start 157.66 98.14) (end 158.459999 98.939999) (width 0.5) (layer "F.Cu") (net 27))
 (segment (start 158.459999 107.4) (end 156.7 107.4) (width 0.5) (layer "F.Cu") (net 27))
 (segment (start 176 75.299) (end 176.5 75.799) (width 0.5) (layer "F.Cu") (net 2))
 (segment (start 175.36 73.02) (end 176 73.66) (width 0.5) (layer "F.Cu") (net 2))
 (segment (start 176.5 75.799) (end 176.5 94.328636) (width 0.5) (layer "F.Cu") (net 2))
 (segment (start 177.671364 95.5) (end 178.5 95.5) (width 0.5) (layer "F.Cu") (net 2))
 (segment (start 176 73.66) (end 176 75.299) (width 0.5) (layer "F.Cu") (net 2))
 (segment (start 176.5 94.328636) (end 177.671364 95.5) (width 0.5) (layer "F.Cu") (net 2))
 (segment (start 131.7 122.7) (end 132.02 123.02) (width 0.5) (layer "F.Cu") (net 43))
 (segment (start 131.7 118.52) (end 131.7 122.7) (width 0.5) (layer "F.Cu") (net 43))
 (segment (start 132.02 123.02) (end 165.15 123.02) (width 0.5) (layer "F.Cu") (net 43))
 (segment (start 165.15 123.02) (end 165.15 121) (width 0.5) (layer "F.Cu") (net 43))
 (segment (start 162.61 72.74) (end 162.61 76.14) (width 0.5) (layer "F.Cu") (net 22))
 (segment (start 162.61 76.14) (end 165.28 78.81) (width 0.5) (layer "F.Cu") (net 22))
 (segment (start 179.2 105.64) (end 176 105.64) (width 0.5) (layer "F.Cu") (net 6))
 (segment (start 173.18 119) (end 173.18 121.15) (width 0.5) (layer "F.Cu") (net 6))
 (segment (start 176 119) (end 173.18 119) (width 0.5) (layer "F.Cu") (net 6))
 (segment (start 176 105.64) (end 176 119) (width 0.5) (layer "F.Cu") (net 6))
 (segment (start 179.2 103.1) (end 175.4 103.1) (width 0.5) (layer "B.Cu") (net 5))
 (segment (start 175.4 103.1) (end 175 103.5) (width 0.5) (layer "B.Cu") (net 5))
 (segment (start 170.5 119.5) (end 170.5 121.01) (width 0.5) (layer "B.Cu") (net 5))
 (segment (start 175 103.5) (end 175 119.5) (width 0.5) (layer "B.Cu") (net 5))
 (segment (start 175 119.5) (end 170.5 119.5) (width 0.5) (layer "B.Cu") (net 5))
 (segment (start 156.42 72.89) (end 138.1 91.21) (width 0.5) (layer "B.Cu") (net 42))
 (segment (start 160.07 72.74) (end 160.07 78.68) (width 0.5) (layer "F.Cu") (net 23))
 (segment (start 152 98.5) (end 152 111.5) (width 0.5) (layer "B.Cu") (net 25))
 (segment (start 152 79) (end 152 98.5) (width 0.5) (layer "B.Cu") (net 25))
 (segment (start 145.15 111.5) (end 145.15 113.44) (width 0.5) (layer "B.Cu") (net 25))
 (segment (start 148.54 98.5) (end 152 98.5) (width 0.5) (layer "B.Cu") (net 25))
 (segment (start 155.12 78.81) (end 152.19 78.81) (width 0.5) (layer "B.Cu") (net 25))
 (segment (start 152.86 121.15) (end 145.15 113.44) (width 0.5) (layer "B.Cu") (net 25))
 (segment (start 152 111.5) (end 145.15 111.5) (width 0.5) (layer "B.Cu") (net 25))
 (segment (start 152.19 78.81) (end 152 79) (width 0.5) (layer "B.Cu") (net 25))
 (segment (start 145.15 113.44) (end 131.7 113.44) (width 0.5) (layer "B.Cu") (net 25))
 (segment (start 143.72 98.24) (end 143.46 98.5) (width 0.5) (layer "F.Cu") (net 41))
 (segment (start 143.72 72.89) (end 143.72 98.24) (width 0.5) (layer "F.Cu") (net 41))
 (segment (start 151.5 75.59) (end 151.5 104.26) (width 0.5) (layer "F.Cu") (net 37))
 (segment (start 151.5 104.26) (end 148.74 107.02) (width 0.5) (layer "F.Cu") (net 37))
 (segment (start 148.8 72.89) (end 151.5 75.59) (width 0.5) (layer "F.Cu") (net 37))
 (segment (start 181.72 110.72) (end 182 111) (width 0.5) (layer "F.Cu") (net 8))
 (segment (start 182 117.41) (end 178.26 121.15) (width 0.5) (layer "F.Cu") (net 8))
 (segment (start 182 111) (end 182 117.41) (width 0.5) (layer "F.Cu") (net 8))
 (segment (start 179.2 110.72) (end 181.72 110.72) (width 0.5) (layer "F.Cu") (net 8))
 (segment (start 146.26 72.89) (end 146.26 98.24) (width 0.5) (layer "F.Cu") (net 40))
 (segment (start 146.26 98.24) (end 146 98.5) (width 0.5) (layer "F.Cu") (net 40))
 (segment (start 135.25 91.52) (end 134.05 91.52) (width 0.5) (layer "B.Cu") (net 36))
 (segment (start 153.88 72.89) (end 135.25 91.52) (width 0.5) (layer "B.Cu") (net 36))
 (segment (start 178.7 73.02) (end 179 73.32) (width 0.5) (layer "F.Cu") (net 1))
 (segment (start 179 73.32) (end 179 92.74) (width 0.5) (layer "F.Cu") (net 1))
 (segment (start 179 92.74) (end 179.2 92.94) (width 0.5) (layer "F.Cu") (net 1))
 (segment (start 133.02 88.5) (end 130 91.52) (width 0.5) (layer "B.Cu") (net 9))
 (segment (start 151.34 72.89) (end 135.73 88.5) (width 0.5) (layer "B.Cu") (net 9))
 (segment (start 135.73 88.5) (end 133.02 88.5) (width 0.5) (layer "B.Cu") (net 9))
 (segment (start 179.2 108.18) (end 177 108.18) (width 0.5) (layer "F.Cu") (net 7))
 (segment (start 177 108.18) (end 177 119.87) (width 0.5) (layer "F.Cu") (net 7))
 (segment (start 177 119.87) (end 175.72 121.15) (width 0.5) (layer "F.Cu") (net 7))
 (segment (start 173.75 76) (end 175.5 76) (width 0.5) (layer "F.Cu") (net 3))
 (segment (start 175.5 76) (end 175.5 94.32) (width 0.5) (layer "F.Cu") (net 3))
 (segment (start 175.5 94.32) (end 179.2 98.02) (width 0.5) (layer "F.Cu") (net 3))
 (segment (start 170.64 72.89) (end 173.75 76) (width 0.5) (layer "F.Cu") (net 3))
 (segment (start 171.45 76.5) (end 176.5 76.5) (width 0.5) (layer "B.Cu") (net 4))
 (segment (start 176.5 76.5) (end 176.5 97.86) (width 0.5) (layer "B.Cu") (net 4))
 (segment (start 167.69 72.74) (end 171.45 76.5) (width 0.5) (layer "B.Cu") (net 4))
 (segment (start 176.5 97.86) (end 179.2 100.56) (width 0.5) (layer "B.Cu") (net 4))
 (segment (start 165.15 72.74) (end 165.15 76.14) (width 0.5) (layer "F.Cu") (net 21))
 (segment (start 165.15 76.14) (end 167.82 78.81) (width 0.5) (layer "F.Cu") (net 21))
 (segment (start 130.38 77.545) (end 130.38 83.52) (width 0.5) (layer "F.Cu") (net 10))
 (segment (start 134.05 81.05) (end 134.05 83.9) (width 0.5) (layer "F.Cu") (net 35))
 (segment (start 132.92 77.545) (end 132.92 79.92) (width 0.5) (layer "F.Cu") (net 35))
 (segment (start 132.92 79.92) (end 134.05 81.05) (width 0.5) (layer "F.Cu") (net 35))
 (segment (start 138 77.545) (end 138 83.8) (width 0.5) (layer "F.Cu") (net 34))
 (segment (start 162.74 86.43) (end 162.74 90.52) (width 0.5) (layer "F.Cu") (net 14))
 (segment (start 152.6 92.4) (end 172.9 92.4) (width 0.5) (layer "F.Cu") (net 24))
 (segment (start 157.66 76.16) (end 157.5 76) (width 0.5) (layer "F.Cu") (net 24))
 (segment (start 152.5 76) (end 152.5 92.3) (width 0.5) (layer "F.Cu") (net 24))
 (segment (start 157.5 76) (end 152.5 76) (width 0.5) (layer "F.Cu") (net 24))
 (segment (start 172.9 90.52) (end 172.9 92.4) (width 0.5) (layer "F.Cu") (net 24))
 (segment (start 157.66 78.81) (end 157.66 76.16) (width 0.5) (layer "F.Cu") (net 24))
 (segment (start 152.5 92.3) (end 152.6 92.4) (width 0.5) (layer "F.Cu") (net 24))
 (segment (start 160.2 86.43) (end 160.2 90.52) (width 0.5) (layer "F.Cu") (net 13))
 (segment (start 157.66 86.43) (end 157.66 90.52) (width 0.5) (layer "F.Cu") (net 12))
 (segment (start 165.28 86.43) (end 165.28 90.52) (width 0.5) (layer "F.Cu") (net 15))
 (segment (start 167.82 86.43) (end 167.82 90.52) (width 0.5) (layer "F.Cu") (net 16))
 (segment (start 155.12 86.43) (end 155.12 90.52) (width 0.5) (layer "F.Cu") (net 11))
 (segment (start 170.36 86.43) (end 170.36 90.52) (width 0.5) (layer "F.Cu") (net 17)))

